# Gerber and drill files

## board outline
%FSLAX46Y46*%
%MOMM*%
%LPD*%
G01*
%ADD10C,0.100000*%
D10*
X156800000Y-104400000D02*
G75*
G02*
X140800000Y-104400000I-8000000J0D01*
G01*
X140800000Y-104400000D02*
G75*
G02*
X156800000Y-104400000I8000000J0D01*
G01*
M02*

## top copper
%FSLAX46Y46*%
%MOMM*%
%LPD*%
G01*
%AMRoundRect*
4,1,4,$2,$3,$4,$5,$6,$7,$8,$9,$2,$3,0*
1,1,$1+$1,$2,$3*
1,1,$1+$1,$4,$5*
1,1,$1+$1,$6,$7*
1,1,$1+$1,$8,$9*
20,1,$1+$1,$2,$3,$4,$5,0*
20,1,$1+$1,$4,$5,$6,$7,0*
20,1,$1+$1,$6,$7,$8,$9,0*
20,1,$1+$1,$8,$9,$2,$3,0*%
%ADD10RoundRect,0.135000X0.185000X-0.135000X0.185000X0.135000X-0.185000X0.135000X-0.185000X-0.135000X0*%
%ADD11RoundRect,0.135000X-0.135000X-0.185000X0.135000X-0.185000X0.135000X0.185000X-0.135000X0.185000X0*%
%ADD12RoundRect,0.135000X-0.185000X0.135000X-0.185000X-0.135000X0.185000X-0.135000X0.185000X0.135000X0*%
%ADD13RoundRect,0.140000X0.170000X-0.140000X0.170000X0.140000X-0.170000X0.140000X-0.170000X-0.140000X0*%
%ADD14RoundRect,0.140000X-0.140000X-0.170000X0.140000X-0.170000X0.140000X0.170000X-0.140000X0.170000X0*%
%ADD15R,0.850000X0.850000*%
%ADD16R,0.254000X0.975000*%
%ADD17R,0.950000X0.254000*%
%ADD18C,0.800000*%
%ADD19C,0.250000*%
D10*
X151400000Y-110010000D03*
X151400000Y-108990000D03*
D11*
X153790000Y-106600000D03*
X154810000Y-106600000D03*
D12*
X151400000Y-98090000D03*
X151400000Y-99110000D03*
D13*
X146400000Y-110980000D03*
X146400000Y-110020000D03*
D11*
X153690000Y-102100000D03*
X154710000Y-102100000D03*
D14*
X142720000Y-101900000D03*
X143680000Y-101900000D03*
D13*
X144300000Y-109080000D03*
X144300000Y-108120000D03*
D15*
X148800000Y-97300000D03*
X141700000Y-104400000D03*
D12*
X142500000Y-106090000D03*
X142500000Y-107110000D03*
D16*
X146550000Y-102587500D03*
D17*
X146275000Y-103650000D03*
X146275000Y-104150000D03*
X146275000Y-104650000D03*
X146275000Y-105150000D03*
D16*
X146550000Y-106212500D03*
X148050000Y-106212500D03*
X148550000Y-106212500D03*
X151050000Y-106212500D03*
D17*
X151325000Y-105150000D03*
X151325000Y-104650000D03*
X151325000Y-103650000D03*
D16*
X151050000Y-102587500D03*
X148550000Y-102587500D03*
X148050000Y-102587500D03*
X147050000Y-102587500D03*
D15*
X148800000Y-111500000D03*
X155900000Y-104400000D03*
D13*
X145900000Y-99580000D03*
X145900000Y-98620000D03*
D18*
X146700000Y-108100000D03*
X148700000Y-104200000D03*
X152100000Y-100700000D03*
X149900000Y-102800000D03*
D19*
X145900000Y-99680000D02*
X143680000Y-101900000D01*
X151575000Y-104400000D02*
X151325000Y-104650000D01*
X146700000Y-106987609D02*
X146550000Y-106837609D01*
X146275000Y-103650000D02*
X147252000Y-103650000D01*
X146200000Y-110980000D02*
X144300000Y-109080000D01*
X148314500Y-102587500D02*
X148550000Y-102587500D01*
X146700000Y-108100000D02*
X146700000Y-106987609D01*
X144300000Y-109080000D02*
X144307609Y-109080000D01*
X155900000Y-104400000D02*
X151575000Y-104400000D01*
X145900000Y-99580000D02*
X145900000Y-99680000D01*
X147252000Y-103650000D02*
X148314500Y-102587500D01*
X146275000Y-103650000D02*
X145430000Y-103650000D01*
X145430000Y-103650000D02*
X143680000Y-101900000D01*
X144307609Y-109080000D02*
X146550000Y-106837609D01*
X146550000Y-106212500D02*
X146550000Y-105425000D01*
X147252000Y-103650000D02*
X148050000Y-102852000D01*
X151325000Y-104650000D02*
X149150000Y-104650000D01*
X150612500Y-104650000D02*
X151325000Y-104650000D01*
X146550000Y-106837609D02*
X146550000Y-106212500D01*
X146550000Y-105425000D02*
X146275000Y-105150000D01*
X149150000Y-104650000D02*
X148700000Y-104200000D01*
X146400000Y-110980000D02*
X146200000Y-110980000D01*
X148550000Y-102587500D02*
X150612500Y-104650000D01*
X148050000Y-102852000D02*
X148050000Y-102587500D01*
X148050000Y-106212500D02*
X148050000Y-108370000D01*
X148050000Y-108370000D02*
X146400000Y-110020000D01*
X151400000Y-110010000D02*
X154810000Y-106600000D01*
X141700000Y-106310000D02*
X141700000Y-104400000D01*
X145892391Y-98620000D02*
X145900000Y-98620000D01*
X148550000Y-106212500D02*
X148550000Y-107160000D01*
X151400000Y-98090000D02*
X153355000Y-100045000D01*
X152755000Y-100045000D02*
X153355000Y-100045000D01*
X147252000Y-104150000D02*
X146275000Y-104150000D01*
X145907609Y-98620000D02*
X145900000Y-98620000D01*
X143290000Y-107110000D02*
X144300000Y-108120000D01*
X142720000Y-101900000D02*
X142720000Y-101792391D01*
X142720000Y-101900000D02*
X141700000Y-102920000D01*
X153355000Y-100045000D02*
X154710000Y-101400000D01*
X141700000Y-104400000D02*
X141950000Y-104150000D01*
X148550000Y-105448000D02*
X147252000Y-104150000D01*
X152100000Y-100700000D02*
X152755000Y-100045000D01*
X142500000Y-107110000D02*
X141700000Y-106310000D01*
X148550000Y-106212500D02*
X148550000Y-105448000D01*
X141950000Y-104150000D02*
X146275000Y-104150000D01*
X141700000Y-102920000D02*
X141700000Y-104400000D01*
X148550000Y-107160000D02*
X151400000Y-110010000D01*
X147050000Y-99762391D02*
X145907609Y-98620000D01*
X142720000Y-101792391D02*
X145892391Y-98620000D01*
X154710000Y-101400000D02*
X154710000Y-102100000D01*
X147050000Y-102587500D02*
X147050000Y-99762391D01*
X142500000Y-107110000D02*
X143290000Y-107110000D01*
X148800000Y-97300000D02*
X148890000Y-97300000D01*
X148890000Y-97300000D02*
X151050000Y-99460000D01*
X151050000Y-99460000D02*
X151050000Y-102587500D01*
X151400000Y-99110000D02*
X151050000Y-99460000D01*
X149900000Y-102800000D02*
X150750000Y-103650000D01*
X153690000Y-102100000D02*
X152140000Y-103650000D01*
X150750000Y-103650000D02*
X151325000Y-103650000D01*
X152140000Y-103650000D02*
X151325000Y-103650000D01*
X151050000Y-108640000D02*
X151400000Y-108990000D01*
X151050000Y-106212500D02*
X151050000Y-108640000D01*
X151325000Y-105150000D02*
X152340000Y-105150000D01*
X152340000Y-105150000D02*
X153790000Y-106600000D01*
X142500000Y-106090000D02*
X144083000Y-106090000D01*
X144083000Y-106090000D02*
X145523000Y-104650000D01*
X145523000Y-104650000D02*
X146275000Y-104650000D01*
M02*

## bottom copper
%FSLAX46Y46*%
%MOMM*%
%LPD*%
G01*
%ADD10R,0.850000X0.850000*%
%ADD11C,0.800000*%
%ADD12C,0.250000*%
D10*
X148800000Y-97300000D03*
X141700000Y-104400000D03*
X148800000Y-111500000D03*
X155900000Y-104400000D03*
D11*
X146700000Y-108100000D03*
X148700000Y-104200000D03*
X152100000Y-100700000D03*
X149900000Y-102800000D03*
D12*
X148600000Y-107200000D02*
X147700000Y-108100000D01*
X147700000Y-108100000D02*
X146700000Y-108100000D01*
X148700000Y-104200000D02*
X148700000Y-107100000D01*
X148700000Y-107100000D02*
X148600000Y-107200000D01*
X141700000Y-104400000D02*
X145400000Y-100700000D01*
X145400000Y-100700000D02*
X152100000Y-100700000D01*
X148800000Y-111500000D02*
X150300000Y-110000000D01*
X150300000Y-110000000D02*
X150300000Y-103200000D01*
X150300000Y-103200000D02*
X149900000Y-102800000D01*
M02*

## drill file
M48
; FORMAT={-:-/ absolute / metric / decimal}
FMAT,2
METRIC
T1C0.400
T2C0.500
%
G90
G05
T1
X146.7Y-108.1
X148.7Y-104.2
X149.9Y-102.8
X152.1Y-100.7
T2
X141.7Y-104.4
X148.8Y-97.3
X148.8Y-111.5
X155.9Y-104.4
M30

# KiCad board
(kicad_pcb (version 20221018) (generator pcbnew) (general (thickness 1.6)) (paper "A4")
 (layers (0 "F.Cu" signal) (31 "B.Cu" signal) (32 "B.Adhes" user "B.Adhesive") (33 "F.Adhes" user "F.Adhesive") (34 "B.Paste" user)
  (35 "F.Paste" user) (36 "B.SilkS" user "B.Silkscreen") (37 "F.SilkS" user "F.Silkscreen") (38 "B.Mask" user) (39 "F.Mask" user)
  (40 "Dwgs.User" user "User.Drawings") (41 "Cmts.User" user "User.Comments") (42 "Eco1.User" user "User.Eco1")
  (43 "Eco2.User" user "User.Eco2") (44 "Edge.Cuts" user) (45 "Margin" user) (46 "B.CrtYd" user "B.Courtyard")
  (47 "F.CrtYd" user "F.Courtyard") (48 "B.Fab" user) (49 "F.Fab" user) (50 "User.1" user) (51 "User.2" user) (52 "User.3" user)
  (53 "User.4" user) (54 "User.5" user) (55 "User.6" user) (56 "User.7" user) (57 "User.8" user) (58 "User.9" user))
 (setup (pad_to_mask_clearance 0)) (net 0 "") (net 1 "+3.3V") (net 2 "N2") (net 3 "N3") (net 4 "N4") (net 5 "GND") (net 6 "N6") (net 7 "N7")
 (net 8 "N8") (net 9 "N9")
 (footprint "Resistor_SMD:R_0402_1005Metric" (layer "F.Cu") (at 151.4 109.5 90)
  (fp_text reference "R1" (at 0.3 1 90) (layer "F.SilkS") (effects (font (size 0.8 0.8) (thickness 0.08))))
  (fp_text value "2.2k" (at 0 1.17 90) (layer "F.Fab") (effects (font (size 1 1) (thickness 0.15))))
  (pad "1" smd roundrect (at -0.51 0 90) (size 0.54 0.64) (layers "F.Cu" "F.Paste" "F.Mask") (roundrect_rratio 0.25) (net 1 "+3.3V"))
  (pad "2" smd roundrect (at 0.51 0 90) (size 0.54 0.64) (layers "F.Cu" "F.Paste" "F.Mask") (roundrect_rratio 0.25) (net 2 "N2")))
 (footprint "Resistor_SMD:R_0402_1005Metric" (layer "F.Cu") (at 154.3 106.6)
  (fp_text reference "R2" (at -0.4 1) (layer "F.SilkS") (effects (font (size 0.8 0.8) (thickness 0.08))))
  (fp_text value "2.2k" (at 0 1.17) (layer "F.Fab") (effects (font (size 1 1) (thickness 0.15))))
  (pad "1" smd roundrect (at -0.51 0) (size 0.54 0.64) (layers "F.Cu" "F.Paste" "F.Mask") (roundrect_rratio 0.25) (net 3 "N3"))
  (pad "2" smd roundrect (at 0.51 0) (size 0.54 0.64) (layers "F.Cu" "F.Paste" "F.Mask") (roundrect_rratio 0.25) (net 1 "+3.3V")))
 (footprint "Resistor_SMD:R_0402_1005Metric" (layer "F.Cu") (at 151.4 98.6 -90)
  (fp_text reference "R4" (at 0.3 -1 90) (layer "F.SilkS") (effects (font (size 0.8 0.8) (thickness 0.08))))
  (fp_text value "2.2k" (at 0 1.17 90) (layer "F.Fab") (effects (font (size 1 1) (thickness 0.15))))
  (pad "1" smd roundrect (at -0.51 0 270) (size 0.54 0.64) (layers "F.Cu" "F.Paste" "F.Mask") (roundrect_rratio 0.25) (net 1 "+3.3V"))
  (pad "2" smd roundrect (at 0.51 0 270) (size 0.54 0.64) (layers "F.Cu" "F.Paste" "F.Mask") (roundrect_rratio 0.25) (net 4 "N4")))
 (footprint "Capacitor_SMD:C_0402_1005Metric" (layer "F.Cu") (at 146.4 110.5 90)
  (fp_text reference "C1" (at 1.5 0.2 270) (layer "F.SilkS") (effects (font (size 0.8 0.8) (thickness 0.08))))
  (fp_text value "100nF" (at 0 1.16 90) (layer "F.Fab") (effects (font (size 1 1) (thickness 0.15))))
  (pad "1" smd roundrect (at -0.48 0 90) (size 0.56 0.62) (layers "F.Cu" "F.Paste" "F.Mask") (roundrect_rratio 0.25) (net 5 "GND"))
  (pad "2" smd roundrect (at 0.48 0 90) (size 0.56 0.62) (layers "F.Cu" "F.Paste" "F.Mask") (roundrect_rratio 0.25) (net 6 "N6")))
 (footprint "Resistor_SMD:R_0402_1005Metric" (layer "F.Cu") (at 154.2 102.1)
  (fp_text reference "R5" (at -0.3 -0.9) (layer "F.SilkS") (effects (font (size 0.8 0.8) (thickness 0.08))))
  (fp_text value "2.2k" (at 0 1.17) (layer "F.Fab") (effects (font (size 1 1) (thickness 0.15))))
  (pad "1" smd roundrect (at -0.51 0) (size 0.54 0.64) (layers "F.Cu" "F.Paste" "F.Mask") (roundrect_rratio 0.25) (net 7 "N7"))
  (pad "2" smd roundrect (at 0.51 0) (size 0.54 0.64) (layers "F.Cu" "F.Paste" "F.Mask") (roundrect_rratio 0.25) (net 1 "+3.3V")))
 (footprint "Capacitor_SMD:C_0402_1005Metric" (layer "F.Cu") (at 143.2 101.9)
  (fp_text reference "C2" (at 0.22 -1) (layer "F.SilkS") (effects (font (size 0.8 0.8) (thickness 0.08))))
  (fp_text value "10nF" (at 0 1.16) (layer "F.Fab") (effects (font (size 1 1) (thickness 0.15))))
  (pad "1" smd roundrect (at -0.48 0) (size 0.56 0.62) (layers "F.Cu" "F.Paste" "F.Mask") (roundrect_rratio 0.25) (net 1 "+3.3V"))
  (pad "2" smd roundrect (at 0.48 0) (size 0.56 0.62) (layers "F.Cu" "F.Paste" "F.Mask") (roundrect_rratio 0.25) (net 5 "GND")))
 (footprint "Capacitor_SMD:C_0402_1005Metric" (layer "F.Cu") (at 144.3 108.6 90)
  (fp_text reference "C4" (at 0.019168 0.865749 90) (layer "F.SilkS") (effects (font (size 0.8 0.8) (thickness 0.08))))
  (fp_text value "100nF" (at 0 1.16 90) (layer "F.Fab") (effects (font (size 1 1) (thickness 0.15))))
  (pad "1" smd roundrect (at -0.48 0 90) (size 0.56 0.62) (layers "F.Cu" "F.Paste" "F.Mask") (roundrect_rratio 0.25) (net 5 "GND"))
  (pad "2" smd roundrect (at 0.48 0 90) (size 0.56 0.62) (layers "F.Cu" "F.Paste" "F.Mask") (roundrect_rratio 0.25) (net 1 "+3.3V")))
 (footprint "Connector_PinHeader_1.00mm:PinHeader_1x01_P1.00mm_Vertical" (layer "F.Cu") (at 148.8 97.3 180)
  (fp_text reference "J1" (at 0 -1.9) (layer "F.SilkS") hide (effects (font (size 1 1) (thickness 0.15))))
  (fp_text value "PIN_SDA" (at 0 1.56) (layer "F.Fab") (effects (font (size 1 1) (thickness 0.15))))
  (pad "1" thru_hole rect (at 0 0 180) (size 0.85 0.85) (drill 0.5) (layers "*.Cu" "*.Mask") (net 4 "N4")))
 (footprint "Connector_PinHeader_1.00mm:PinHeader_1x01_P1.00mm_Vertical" (layer "F.Cu") (at 141.7 104.4 -90)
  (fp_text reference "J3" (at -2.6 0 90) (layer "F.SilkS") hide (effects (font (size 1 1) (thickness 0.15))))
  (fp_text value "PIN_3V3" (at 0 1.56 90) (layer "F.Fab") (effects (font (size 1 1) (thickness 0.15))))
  (pad "1" thru_hole rect (at 0 0 270) (size 0.85 0.85) (drill 0.5) (layers "*.Cu" "*.Mask") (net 1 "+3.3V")))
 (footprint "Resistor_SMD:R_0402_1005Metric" (layer "F.Cu") (at 142.5 106.6 -90)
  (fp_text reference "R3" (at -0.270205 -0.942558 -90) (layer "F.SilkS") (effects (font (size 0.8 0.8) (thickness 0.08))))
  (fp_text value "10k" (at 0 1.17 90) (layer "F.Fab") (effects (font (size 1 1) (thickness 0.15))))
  (pad "1" smd roundrect (at -0.51 0 270) (size 0.54 0.64) (layers "F.Cu" "F.Paste" "F.Mask") (roundrect_rratio 0.25) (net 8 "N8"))
  (pad "2" smd roundrect (at 0.51 0 270) (size 0.54 0.64) (layers "F.Cu" "F.Paste" "F.Mask") (roundrect_rratio 0.25) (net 1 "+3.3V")))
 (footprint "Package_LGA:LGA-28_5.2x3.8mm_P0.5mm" (layer "F.Cu") (at 148.8 104.4)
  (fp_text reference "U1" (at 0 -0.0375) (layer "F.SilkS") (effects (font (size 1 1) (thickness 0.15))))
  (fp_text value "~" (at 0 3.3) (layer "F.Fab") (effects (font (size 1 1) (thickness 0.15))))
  (pad "1" smd rect (at -2.25 -1.8125) (size 0.254 0.975) (layers "F.Cu" "F.Paste" "F.Mask") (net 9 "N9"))
  (pad "2" smd rect (at -2.525 -0.75 90) (size 0.254 0.95) (layers "F.Cu" "F.Paste" "F.Mask") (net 5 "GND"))
  (pad "3" smd rect (at -2.525 -0.25 90) (size 0.254 0.95) (layers "F.Cu" "F.Paste" "F.Mask") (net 1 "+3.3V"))
  (pad "4" smd rect (at -2.525 0.25 90) (size 0.254 0.95) (layers "F.Cu" "F.Paste" "F.Mask") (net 8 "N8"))
  (pad "5" smd rect (at -2.525 0.75 90) (size 0.254 0.95) (layers "F.Cu" "F.Paste" "F.Mask") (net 5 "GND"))
  (pad "6" smd rect (at -2.25 1.8125) (size 0.254 0.975) (layers "F.Cu" "F.Paste" "F.Mask") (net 5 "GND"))
  (pad "9" smd rect (at -0.75 1.8125) (size 0.254 0.975) (layers "F.Cu" "F.Paste" "F.Mask") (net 6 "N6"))
  (pad "10" smd rect (at -0.25 1.8125) (size 0.254 0.975) (layers "F.Cu" "F.Paste" "F.Mask") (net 1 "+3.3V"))
  (pad "15" smd rect (at 2.25 1.8125) (size 0.254 0.975) (layers "F.Cu" "F.Paste" "F.Mask") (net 2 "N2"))
  (pad "16" smd rect (at 2.525 0.75 90) (size 0.254 0.95) (layers "F.Cu" "F.Paste" "F.Mask") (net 3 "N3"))
  (pad "17" smd rect (at 2.525 0.25 90) (size 0.254 0.95) (layers "F.Cu" "F.Paste" "F.Mask") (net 5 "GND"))
  (pad "19" smd rect (at 2.525 -0.75 90) (size 0.254 0.95) (layers "F.Cu" "F.Paste" "F.Mask") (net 7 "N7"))
  (pad "20" smd rect (at 2.25 -1.8125) (size 0.254 0.975) (layers "F.Cu" "F.Paste" "F.Mask") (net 4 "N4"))
  (pad "25" smd rect (at -0.25 -1.8125) (size 0.254 0.975) (layers "F.Cu" "F.Paste" "F.Mask") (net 5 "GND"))
  (pad "26" smd rect (at -0.75 -1.8125) (size 0.254 0.975) (layers "F.Cu" "F.Paste" "F.Mask") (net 5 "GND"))
  (pad "28" smd rect (at -1.75 -1.8125) (size 0.254 0.975) (layers "F.Cu" "F.Paste" "F.Mask") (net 1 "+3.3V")))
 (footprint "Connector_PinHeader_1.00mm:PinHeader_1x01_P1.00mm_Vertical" (layer "F.Cu") (at 148.8 111.5)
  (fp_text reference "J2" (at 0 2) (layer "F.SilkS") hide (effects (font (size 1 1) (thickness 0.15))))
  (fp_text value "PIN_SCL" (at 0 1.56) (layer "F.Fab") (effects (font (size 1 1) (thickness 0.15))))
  (pad "1" thru_hole rect (at 0 0) (size 0.85 0.85) (drill 0.5) (layers "*.Cu" "*.Mask") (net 7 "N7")))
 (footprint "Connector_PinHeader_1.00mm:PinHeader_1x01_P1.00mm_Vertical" (layer "F.Cu") (at 155.9 104.4 90)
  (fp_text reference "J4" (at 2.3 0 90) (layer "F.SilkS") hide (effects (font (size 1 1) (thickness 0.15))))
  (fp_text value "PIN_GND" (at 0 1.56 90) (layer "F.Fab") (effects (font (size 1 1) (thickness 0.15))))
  (pad "1" thru_hole rect (at 0 0 90) (size 0.85 0.85) (drill 0.5) (layers "*.Cu" "*.Mask") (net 5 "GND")))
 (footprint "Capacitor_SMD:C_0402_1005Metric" (layer "F.Cu") (at 145.9 99.1 90)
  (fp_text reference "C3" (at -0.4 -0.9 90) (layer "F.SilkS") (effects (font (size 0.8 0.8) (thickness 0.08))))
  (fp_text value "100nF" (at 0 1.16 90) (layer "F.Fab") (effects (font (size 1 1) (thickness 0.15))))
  (pad "1" smd roundrect (at -0.48 0 90) (size 0.56 0.62) (layers "F.Cu" "F.Paste" "F.Mask") (roundrect_rratio 0.25) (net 5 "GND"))
  (pad "2" smd roundrect (at 0.48 0 90) (size 0.56 0.62) (layers "F.Cu" "F.Paste" "F.Mask") (roundrect_rratio 0.25) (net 1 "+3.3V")))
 (gr_circle (center 148.8 104.4) (end 156.8 104.4) (stroke (width 0.1) (type default)) (fill none) (layer "Edge.Cuts"))
 (segment (start 145.9 99.68) (end 143.68 101.9) (width 0.25) (layer "F.Cu") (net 5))
 (segment (start 151.575 104.4) (end 151.325 104.65) (width 0.25) (layer "F.Cu") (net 5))
 (segment (start 146.7 106.987609) (end 146.55 106.837609) (width 0.25) (layer "F.Cu") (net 5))
 (segment (start 146.275 103.65) (end 147.252 103.65) (width 0.25) (layer "F.Cu") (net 5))
 (segment (start 146.2 110.98) (end 144.3 109.08) (width 0.25) (layer "F.Cu") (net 5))
 (segment (start 148.3145 102.5875) (end 148.55 102.5875) (width 0.25) (layer "F.Cu") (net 5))
 (segment (start 146.7 108.1) (end 146.7 106.987609) (width 0.25) (layer "F.Cu") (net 5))
 (segment (start 144.3 109.08) (end 144.307609 109.08) (width 0.25) (layer "F.Cu") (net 5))
 (segment (start 155.9 104.4) (end 151.575 104.4) (width 0.25) (layer "F.Cu") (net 5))
 (segment (start 145.9 99.58) (end 145.9 99.68) (width 0.25) (layer "F.Cu") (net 5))
 (segment (start 147.252 103.65) (end 148.3145 102.5875) (width 0.25) (layer "F.Cu") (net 5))
 (segment (start 146.275 103.65) (end 145.43 103.65) (width 0.25) (layer "F.Cu") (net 5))
 (segment (start 145.43 103.65) (end 143.68 101.9) (width 0.25) (layer "F.Cu") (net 5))
 (segment (start 144.307609 109.08) (end 146.55 106.837609) (width 0.25) (layer "F.Cu") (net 5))
 (segment (start 146.55 106.2125) (end 146.55 105.425) (width 0.25) (layer "F.Cu") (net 5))
 (segment (start 147.252 103.65) (end 148.05 102.852) (width 0.25) (layer "F.Cu") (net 5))
 (segment (start 151.325 104.65) (end 149.15 104.65) (width 0.25) (layer "F.Cu") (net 5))
 (segment (start 150.6125 104.65) (end 151.325 104.65) (width 0.25) (layer "F.Cu") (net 5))
 (segment (start 146.55 106.837609) (end 146.55 106.2125) (width 0.25) (layer "F.Cu") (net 5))
 (segment (start 146.55 105.425) (end 146.275 105.15) (width 0.25) (layer "F.Cu") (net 5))
 (segment (start 149.15 104.65) (end 148.7 104.2) (width 0.25) (layer "F.Cu") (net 5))
 (segment (start 146.4 110.98) (end 146.2 110.98) (width 0.25) (layer "F.Cu") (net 5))
 (segment (start 148.55 102.5875) (end 150.6125 104.65) (width 0.25) (layer "F.Cu") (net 5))
 (segment (start 148.05 102.852) (end 148.05 102.5875) (width 0.25) (layer "F.Cu") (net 5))
 (via (at 146.7 108.1) (size 0.8) (drill 0.4) (layers "F.Cu" "B.Cu") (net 5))
 (via (at 148.7 104.2) (size 0.8) (drill 0.4) (layers "F.Cu" "B.Cu") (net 5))
 (segment (start 148.6 107.2) (end 147.7 108.1) (width 0.25) (layer "B.Cu") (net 5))
 (segment (start 147.7 108.1) (end 146.7 108.1) (width 0.25) (layer "B.Cu") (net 5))
 (segment (start 148.7 104.2) (end 148.7 107.1) (width 0.25) (layer "B.Cu") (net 5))
 (segment (start 148.7 107.1) (end 148.6 107.2) (width 0.25) (layer "B.Cu") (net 5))
 (segment (start 148.05 106.2125) (end 148.05 108.37) (width 0.25) (layer "F.Cu") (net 6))
 (segment (start 148.05 108.37) (end 146.4 110.02) (width 0.25) (layer "F.Cu") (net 6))
 (segment (start 151.4 110.01) (end 154.81 106.6) (width 0.25) (layer "F.Cu") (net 1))
 (segment (start 141.7 106.31) (end 141.7 104.4) (width 0.25) (layer "F.Cu") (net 1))
 (segment (start 145.892391 98.62) (end 145.9 98.62) (width 0.25) (layer "F.Cu") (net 1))
 (segment (start 148.55 106.2125) (end 148.55 107.16) (width 0.25) (layer "F.Cu") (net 1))
 (segment (start 151.4 98.09) (end 153.355 100.045) (width 0.25) (layer "F.Cu") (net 1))
 (segment (start 152.755 100.045) (end 153.355 100.045) (width 0.25) (layer "F.Cu") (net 1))
 (segment (start 147.252 104.15) (end 146.275 104.15) (width 0.25) (layer "F.Cu") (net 1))
 (segment (start 145.907609 98.62) (end 145.9 98.62) (width 0.25) (layer "F.Cu") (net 1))
 (segment (start 143.29 107.11) (end 144.3 108.12) (width 0.25) (layer "F.Cu") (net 1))
 (segment (start 142.72 101.9) (end 142.72 101.792391) (width 0.25) (layer "F.Cu") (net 1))
 (segment (start 142.72 101.9) (end 141.7 102.92) (width 0.25) (layer "F.Cu") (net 1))
 (segment (start 153.355 100.045) (end 154.71 101.4) (width 0.25) (layer "F.Cu") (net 1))
 (segment (start 141.7 104.4) (end 141.95 104.15) (width 0.25) (layer "F.Cu") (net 1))
 (segment (start 148.55 105.448) (end 147.252 104.15) (width 0.25) (layer "F.Cu") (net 1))
 (segment (start 152.1 100.7) (end 152.755 100.045) (width 0.25) (layer "F.Cu") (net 1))
 (segment (start 142.5 107.11) (end 141.7 106.31) (width 0.25) (layer "F.Cu") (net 1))
 (segment (start 148.55 106.2125) (end 148.55 105.448) (width 0.25) (layer "F.Cu") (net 1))
 (segment (start 141.95 104.15) (end 146.275 104.15) (width 0.25) (layer "F.Cu") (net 1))
 (segment (start 141.7 102.92) (end 141.7 104.4) (width 0.25) (layer "F.Cu") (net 1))
 (segment (start 148.55 107.16) (end 151.4 110.01) (width 0.25) (layer "F.Cu") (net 1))
 (segment (start 147.05 99.762391) (end 145.907609 98.62) (width 0.25) (layer "F.Cu") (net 1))
 (segment (start 142.72 101.792391) (end 145.892391 98.62) (width 0.25) (layer "F.Cu") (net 1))
 (segment (start 154.71 101.4) (end 154.71 102.1) (width 0.25) (layer "F.Cu") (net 1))
 (segment (start 147.05 102.5875) (end 147.05 99.762391) (width 0.25) (layer "F.Cu") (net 1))
 (segment (start 142.5 107.11) (end 143.29 107.11) (width 0.25) (layer "F.Cu") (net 1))
 (via (at 152.1 100.7) (size 0.8) (drill 0.4) (layers "F.Cu" "B.Cu") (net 1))
 (segment (start 141.7 104.4) (end 145.4 100.7) (width 0.25) (layer "B.Cu") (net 1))
 (segment (start 145.4 100.7) (end 152.1 100.7) (width 0.25) (layer "B.Cu") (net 1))
 (segment (start 148.8 97.3) (end 148.89 97.3) (width 0.25) (layer "F.Cu") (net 4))
 (segment (start 148.89 97.3) (end 151.05 99.46) (width 0.25) (layer "F.Cu") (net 4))
 (segment (start 151.05 99.46) (end 151.05 102.5875) (width 0.25) (layer "F.Cu") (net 4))
 (segment (start 151.4 99.11) (end 151.05 99.46) (width 0.25) (layer "F.Cu") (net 4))
 (segment (start 149.9 102.8) (end 150.75 103.65) (width 0.25) (layer "F.Cu") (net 7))
 (segment (start 153.69 102.1) (end 152.14 103.65) (width 0.25) (layer "F.Cu") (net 7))
 (segment (start 150.75 103.65) (end 151.325 103.65) (width 0.25) (layer "F.Cu") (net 7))
 (segment (start 152.14 103.65) (end 151.325 103.65) (width 0.25) (layer "F.Cu") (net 7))
 (via (at 149.9 102.8) (size 0.8) (drill 0.4) (layers "F.Cu" "B.Cu") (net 7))
 (segment (start 148.8 111.5) (end 150.3 110) (width 0.25) (layer "B.Cu") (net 7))
 (segment (start 150.3 110) (end 150.3 103.2) (width 0.25) (layer "B.Cu") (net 7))
 (segment (start 150.3 103.2) (end 149.9 102.8) (width 0.25) (layer "B.Cu") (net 7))
 (segment (start 151.05 108.64) (end 151.4 108.99) (width 0.25) (layer "F.Cu") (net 2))
 (segment (start 151.05 106.2125) (end 151.05 108.64) (width 0.25) (layer "F.Cu") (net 2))
 (segment (start 151.325 105.15) (end 152.34 105.15) (width 0.25) (layer "F.Cu") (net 3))
 (segment (start 152.34 105.15) (end 153.79 106.6) (width 0.25) (layer "F.Cu") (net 3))
 (segment (start 142.5 106.09) (end 144.083 106.09) (width 0.25) (layer "F.Cu") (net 8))
 (segment (start 144.083 106.09) (end 145.523 104.65) (width 0.25) (layer "F.Cu") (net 8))
 (segment (start 145.523 104.65) (end 146.275 104.65) (width 0.25) (layer "F.Cu") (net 8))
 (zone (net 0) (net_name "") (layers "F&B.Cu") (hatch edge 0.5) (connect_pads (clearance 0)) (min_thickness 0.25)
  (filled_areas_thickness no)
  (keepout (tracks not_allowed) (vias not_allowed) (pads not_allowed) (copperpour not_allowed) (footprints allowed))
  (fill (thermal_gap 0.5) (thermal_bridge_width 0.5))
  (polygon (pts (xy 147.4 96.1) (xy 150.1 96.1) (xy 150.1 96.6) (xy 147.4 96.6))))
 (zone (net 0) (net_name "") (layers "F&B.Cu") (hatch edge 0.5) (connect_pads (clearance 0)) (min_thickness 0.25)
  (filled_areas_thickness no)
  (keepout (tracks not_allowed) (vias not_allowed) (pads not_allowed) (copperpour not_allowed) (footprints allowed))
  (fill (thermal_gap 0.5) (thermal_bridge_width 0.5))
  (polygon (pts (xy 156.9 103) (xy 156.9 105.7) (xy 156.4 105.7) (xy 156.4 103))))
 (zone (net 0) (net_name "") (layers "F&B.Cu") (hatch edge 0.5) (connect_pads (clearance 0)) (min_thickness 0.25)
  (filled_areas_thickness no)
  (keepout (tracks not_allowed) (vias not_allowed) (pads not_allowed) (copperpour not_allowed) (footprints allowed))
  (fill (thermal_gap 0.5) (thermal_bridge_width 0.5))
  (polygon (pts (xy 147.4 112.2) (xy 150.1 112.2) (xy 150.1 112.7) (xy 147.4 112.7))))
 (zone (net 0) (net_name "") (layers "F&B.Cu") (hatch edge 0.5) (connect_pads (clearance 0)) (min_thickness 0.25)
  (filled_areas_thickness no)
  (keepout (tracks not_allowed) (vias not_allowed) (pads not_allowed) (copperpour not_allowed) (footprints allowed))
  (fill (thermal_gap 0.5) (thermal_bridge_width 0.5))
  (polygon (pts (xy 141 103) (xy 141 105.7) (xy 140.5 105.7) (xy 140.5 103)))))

